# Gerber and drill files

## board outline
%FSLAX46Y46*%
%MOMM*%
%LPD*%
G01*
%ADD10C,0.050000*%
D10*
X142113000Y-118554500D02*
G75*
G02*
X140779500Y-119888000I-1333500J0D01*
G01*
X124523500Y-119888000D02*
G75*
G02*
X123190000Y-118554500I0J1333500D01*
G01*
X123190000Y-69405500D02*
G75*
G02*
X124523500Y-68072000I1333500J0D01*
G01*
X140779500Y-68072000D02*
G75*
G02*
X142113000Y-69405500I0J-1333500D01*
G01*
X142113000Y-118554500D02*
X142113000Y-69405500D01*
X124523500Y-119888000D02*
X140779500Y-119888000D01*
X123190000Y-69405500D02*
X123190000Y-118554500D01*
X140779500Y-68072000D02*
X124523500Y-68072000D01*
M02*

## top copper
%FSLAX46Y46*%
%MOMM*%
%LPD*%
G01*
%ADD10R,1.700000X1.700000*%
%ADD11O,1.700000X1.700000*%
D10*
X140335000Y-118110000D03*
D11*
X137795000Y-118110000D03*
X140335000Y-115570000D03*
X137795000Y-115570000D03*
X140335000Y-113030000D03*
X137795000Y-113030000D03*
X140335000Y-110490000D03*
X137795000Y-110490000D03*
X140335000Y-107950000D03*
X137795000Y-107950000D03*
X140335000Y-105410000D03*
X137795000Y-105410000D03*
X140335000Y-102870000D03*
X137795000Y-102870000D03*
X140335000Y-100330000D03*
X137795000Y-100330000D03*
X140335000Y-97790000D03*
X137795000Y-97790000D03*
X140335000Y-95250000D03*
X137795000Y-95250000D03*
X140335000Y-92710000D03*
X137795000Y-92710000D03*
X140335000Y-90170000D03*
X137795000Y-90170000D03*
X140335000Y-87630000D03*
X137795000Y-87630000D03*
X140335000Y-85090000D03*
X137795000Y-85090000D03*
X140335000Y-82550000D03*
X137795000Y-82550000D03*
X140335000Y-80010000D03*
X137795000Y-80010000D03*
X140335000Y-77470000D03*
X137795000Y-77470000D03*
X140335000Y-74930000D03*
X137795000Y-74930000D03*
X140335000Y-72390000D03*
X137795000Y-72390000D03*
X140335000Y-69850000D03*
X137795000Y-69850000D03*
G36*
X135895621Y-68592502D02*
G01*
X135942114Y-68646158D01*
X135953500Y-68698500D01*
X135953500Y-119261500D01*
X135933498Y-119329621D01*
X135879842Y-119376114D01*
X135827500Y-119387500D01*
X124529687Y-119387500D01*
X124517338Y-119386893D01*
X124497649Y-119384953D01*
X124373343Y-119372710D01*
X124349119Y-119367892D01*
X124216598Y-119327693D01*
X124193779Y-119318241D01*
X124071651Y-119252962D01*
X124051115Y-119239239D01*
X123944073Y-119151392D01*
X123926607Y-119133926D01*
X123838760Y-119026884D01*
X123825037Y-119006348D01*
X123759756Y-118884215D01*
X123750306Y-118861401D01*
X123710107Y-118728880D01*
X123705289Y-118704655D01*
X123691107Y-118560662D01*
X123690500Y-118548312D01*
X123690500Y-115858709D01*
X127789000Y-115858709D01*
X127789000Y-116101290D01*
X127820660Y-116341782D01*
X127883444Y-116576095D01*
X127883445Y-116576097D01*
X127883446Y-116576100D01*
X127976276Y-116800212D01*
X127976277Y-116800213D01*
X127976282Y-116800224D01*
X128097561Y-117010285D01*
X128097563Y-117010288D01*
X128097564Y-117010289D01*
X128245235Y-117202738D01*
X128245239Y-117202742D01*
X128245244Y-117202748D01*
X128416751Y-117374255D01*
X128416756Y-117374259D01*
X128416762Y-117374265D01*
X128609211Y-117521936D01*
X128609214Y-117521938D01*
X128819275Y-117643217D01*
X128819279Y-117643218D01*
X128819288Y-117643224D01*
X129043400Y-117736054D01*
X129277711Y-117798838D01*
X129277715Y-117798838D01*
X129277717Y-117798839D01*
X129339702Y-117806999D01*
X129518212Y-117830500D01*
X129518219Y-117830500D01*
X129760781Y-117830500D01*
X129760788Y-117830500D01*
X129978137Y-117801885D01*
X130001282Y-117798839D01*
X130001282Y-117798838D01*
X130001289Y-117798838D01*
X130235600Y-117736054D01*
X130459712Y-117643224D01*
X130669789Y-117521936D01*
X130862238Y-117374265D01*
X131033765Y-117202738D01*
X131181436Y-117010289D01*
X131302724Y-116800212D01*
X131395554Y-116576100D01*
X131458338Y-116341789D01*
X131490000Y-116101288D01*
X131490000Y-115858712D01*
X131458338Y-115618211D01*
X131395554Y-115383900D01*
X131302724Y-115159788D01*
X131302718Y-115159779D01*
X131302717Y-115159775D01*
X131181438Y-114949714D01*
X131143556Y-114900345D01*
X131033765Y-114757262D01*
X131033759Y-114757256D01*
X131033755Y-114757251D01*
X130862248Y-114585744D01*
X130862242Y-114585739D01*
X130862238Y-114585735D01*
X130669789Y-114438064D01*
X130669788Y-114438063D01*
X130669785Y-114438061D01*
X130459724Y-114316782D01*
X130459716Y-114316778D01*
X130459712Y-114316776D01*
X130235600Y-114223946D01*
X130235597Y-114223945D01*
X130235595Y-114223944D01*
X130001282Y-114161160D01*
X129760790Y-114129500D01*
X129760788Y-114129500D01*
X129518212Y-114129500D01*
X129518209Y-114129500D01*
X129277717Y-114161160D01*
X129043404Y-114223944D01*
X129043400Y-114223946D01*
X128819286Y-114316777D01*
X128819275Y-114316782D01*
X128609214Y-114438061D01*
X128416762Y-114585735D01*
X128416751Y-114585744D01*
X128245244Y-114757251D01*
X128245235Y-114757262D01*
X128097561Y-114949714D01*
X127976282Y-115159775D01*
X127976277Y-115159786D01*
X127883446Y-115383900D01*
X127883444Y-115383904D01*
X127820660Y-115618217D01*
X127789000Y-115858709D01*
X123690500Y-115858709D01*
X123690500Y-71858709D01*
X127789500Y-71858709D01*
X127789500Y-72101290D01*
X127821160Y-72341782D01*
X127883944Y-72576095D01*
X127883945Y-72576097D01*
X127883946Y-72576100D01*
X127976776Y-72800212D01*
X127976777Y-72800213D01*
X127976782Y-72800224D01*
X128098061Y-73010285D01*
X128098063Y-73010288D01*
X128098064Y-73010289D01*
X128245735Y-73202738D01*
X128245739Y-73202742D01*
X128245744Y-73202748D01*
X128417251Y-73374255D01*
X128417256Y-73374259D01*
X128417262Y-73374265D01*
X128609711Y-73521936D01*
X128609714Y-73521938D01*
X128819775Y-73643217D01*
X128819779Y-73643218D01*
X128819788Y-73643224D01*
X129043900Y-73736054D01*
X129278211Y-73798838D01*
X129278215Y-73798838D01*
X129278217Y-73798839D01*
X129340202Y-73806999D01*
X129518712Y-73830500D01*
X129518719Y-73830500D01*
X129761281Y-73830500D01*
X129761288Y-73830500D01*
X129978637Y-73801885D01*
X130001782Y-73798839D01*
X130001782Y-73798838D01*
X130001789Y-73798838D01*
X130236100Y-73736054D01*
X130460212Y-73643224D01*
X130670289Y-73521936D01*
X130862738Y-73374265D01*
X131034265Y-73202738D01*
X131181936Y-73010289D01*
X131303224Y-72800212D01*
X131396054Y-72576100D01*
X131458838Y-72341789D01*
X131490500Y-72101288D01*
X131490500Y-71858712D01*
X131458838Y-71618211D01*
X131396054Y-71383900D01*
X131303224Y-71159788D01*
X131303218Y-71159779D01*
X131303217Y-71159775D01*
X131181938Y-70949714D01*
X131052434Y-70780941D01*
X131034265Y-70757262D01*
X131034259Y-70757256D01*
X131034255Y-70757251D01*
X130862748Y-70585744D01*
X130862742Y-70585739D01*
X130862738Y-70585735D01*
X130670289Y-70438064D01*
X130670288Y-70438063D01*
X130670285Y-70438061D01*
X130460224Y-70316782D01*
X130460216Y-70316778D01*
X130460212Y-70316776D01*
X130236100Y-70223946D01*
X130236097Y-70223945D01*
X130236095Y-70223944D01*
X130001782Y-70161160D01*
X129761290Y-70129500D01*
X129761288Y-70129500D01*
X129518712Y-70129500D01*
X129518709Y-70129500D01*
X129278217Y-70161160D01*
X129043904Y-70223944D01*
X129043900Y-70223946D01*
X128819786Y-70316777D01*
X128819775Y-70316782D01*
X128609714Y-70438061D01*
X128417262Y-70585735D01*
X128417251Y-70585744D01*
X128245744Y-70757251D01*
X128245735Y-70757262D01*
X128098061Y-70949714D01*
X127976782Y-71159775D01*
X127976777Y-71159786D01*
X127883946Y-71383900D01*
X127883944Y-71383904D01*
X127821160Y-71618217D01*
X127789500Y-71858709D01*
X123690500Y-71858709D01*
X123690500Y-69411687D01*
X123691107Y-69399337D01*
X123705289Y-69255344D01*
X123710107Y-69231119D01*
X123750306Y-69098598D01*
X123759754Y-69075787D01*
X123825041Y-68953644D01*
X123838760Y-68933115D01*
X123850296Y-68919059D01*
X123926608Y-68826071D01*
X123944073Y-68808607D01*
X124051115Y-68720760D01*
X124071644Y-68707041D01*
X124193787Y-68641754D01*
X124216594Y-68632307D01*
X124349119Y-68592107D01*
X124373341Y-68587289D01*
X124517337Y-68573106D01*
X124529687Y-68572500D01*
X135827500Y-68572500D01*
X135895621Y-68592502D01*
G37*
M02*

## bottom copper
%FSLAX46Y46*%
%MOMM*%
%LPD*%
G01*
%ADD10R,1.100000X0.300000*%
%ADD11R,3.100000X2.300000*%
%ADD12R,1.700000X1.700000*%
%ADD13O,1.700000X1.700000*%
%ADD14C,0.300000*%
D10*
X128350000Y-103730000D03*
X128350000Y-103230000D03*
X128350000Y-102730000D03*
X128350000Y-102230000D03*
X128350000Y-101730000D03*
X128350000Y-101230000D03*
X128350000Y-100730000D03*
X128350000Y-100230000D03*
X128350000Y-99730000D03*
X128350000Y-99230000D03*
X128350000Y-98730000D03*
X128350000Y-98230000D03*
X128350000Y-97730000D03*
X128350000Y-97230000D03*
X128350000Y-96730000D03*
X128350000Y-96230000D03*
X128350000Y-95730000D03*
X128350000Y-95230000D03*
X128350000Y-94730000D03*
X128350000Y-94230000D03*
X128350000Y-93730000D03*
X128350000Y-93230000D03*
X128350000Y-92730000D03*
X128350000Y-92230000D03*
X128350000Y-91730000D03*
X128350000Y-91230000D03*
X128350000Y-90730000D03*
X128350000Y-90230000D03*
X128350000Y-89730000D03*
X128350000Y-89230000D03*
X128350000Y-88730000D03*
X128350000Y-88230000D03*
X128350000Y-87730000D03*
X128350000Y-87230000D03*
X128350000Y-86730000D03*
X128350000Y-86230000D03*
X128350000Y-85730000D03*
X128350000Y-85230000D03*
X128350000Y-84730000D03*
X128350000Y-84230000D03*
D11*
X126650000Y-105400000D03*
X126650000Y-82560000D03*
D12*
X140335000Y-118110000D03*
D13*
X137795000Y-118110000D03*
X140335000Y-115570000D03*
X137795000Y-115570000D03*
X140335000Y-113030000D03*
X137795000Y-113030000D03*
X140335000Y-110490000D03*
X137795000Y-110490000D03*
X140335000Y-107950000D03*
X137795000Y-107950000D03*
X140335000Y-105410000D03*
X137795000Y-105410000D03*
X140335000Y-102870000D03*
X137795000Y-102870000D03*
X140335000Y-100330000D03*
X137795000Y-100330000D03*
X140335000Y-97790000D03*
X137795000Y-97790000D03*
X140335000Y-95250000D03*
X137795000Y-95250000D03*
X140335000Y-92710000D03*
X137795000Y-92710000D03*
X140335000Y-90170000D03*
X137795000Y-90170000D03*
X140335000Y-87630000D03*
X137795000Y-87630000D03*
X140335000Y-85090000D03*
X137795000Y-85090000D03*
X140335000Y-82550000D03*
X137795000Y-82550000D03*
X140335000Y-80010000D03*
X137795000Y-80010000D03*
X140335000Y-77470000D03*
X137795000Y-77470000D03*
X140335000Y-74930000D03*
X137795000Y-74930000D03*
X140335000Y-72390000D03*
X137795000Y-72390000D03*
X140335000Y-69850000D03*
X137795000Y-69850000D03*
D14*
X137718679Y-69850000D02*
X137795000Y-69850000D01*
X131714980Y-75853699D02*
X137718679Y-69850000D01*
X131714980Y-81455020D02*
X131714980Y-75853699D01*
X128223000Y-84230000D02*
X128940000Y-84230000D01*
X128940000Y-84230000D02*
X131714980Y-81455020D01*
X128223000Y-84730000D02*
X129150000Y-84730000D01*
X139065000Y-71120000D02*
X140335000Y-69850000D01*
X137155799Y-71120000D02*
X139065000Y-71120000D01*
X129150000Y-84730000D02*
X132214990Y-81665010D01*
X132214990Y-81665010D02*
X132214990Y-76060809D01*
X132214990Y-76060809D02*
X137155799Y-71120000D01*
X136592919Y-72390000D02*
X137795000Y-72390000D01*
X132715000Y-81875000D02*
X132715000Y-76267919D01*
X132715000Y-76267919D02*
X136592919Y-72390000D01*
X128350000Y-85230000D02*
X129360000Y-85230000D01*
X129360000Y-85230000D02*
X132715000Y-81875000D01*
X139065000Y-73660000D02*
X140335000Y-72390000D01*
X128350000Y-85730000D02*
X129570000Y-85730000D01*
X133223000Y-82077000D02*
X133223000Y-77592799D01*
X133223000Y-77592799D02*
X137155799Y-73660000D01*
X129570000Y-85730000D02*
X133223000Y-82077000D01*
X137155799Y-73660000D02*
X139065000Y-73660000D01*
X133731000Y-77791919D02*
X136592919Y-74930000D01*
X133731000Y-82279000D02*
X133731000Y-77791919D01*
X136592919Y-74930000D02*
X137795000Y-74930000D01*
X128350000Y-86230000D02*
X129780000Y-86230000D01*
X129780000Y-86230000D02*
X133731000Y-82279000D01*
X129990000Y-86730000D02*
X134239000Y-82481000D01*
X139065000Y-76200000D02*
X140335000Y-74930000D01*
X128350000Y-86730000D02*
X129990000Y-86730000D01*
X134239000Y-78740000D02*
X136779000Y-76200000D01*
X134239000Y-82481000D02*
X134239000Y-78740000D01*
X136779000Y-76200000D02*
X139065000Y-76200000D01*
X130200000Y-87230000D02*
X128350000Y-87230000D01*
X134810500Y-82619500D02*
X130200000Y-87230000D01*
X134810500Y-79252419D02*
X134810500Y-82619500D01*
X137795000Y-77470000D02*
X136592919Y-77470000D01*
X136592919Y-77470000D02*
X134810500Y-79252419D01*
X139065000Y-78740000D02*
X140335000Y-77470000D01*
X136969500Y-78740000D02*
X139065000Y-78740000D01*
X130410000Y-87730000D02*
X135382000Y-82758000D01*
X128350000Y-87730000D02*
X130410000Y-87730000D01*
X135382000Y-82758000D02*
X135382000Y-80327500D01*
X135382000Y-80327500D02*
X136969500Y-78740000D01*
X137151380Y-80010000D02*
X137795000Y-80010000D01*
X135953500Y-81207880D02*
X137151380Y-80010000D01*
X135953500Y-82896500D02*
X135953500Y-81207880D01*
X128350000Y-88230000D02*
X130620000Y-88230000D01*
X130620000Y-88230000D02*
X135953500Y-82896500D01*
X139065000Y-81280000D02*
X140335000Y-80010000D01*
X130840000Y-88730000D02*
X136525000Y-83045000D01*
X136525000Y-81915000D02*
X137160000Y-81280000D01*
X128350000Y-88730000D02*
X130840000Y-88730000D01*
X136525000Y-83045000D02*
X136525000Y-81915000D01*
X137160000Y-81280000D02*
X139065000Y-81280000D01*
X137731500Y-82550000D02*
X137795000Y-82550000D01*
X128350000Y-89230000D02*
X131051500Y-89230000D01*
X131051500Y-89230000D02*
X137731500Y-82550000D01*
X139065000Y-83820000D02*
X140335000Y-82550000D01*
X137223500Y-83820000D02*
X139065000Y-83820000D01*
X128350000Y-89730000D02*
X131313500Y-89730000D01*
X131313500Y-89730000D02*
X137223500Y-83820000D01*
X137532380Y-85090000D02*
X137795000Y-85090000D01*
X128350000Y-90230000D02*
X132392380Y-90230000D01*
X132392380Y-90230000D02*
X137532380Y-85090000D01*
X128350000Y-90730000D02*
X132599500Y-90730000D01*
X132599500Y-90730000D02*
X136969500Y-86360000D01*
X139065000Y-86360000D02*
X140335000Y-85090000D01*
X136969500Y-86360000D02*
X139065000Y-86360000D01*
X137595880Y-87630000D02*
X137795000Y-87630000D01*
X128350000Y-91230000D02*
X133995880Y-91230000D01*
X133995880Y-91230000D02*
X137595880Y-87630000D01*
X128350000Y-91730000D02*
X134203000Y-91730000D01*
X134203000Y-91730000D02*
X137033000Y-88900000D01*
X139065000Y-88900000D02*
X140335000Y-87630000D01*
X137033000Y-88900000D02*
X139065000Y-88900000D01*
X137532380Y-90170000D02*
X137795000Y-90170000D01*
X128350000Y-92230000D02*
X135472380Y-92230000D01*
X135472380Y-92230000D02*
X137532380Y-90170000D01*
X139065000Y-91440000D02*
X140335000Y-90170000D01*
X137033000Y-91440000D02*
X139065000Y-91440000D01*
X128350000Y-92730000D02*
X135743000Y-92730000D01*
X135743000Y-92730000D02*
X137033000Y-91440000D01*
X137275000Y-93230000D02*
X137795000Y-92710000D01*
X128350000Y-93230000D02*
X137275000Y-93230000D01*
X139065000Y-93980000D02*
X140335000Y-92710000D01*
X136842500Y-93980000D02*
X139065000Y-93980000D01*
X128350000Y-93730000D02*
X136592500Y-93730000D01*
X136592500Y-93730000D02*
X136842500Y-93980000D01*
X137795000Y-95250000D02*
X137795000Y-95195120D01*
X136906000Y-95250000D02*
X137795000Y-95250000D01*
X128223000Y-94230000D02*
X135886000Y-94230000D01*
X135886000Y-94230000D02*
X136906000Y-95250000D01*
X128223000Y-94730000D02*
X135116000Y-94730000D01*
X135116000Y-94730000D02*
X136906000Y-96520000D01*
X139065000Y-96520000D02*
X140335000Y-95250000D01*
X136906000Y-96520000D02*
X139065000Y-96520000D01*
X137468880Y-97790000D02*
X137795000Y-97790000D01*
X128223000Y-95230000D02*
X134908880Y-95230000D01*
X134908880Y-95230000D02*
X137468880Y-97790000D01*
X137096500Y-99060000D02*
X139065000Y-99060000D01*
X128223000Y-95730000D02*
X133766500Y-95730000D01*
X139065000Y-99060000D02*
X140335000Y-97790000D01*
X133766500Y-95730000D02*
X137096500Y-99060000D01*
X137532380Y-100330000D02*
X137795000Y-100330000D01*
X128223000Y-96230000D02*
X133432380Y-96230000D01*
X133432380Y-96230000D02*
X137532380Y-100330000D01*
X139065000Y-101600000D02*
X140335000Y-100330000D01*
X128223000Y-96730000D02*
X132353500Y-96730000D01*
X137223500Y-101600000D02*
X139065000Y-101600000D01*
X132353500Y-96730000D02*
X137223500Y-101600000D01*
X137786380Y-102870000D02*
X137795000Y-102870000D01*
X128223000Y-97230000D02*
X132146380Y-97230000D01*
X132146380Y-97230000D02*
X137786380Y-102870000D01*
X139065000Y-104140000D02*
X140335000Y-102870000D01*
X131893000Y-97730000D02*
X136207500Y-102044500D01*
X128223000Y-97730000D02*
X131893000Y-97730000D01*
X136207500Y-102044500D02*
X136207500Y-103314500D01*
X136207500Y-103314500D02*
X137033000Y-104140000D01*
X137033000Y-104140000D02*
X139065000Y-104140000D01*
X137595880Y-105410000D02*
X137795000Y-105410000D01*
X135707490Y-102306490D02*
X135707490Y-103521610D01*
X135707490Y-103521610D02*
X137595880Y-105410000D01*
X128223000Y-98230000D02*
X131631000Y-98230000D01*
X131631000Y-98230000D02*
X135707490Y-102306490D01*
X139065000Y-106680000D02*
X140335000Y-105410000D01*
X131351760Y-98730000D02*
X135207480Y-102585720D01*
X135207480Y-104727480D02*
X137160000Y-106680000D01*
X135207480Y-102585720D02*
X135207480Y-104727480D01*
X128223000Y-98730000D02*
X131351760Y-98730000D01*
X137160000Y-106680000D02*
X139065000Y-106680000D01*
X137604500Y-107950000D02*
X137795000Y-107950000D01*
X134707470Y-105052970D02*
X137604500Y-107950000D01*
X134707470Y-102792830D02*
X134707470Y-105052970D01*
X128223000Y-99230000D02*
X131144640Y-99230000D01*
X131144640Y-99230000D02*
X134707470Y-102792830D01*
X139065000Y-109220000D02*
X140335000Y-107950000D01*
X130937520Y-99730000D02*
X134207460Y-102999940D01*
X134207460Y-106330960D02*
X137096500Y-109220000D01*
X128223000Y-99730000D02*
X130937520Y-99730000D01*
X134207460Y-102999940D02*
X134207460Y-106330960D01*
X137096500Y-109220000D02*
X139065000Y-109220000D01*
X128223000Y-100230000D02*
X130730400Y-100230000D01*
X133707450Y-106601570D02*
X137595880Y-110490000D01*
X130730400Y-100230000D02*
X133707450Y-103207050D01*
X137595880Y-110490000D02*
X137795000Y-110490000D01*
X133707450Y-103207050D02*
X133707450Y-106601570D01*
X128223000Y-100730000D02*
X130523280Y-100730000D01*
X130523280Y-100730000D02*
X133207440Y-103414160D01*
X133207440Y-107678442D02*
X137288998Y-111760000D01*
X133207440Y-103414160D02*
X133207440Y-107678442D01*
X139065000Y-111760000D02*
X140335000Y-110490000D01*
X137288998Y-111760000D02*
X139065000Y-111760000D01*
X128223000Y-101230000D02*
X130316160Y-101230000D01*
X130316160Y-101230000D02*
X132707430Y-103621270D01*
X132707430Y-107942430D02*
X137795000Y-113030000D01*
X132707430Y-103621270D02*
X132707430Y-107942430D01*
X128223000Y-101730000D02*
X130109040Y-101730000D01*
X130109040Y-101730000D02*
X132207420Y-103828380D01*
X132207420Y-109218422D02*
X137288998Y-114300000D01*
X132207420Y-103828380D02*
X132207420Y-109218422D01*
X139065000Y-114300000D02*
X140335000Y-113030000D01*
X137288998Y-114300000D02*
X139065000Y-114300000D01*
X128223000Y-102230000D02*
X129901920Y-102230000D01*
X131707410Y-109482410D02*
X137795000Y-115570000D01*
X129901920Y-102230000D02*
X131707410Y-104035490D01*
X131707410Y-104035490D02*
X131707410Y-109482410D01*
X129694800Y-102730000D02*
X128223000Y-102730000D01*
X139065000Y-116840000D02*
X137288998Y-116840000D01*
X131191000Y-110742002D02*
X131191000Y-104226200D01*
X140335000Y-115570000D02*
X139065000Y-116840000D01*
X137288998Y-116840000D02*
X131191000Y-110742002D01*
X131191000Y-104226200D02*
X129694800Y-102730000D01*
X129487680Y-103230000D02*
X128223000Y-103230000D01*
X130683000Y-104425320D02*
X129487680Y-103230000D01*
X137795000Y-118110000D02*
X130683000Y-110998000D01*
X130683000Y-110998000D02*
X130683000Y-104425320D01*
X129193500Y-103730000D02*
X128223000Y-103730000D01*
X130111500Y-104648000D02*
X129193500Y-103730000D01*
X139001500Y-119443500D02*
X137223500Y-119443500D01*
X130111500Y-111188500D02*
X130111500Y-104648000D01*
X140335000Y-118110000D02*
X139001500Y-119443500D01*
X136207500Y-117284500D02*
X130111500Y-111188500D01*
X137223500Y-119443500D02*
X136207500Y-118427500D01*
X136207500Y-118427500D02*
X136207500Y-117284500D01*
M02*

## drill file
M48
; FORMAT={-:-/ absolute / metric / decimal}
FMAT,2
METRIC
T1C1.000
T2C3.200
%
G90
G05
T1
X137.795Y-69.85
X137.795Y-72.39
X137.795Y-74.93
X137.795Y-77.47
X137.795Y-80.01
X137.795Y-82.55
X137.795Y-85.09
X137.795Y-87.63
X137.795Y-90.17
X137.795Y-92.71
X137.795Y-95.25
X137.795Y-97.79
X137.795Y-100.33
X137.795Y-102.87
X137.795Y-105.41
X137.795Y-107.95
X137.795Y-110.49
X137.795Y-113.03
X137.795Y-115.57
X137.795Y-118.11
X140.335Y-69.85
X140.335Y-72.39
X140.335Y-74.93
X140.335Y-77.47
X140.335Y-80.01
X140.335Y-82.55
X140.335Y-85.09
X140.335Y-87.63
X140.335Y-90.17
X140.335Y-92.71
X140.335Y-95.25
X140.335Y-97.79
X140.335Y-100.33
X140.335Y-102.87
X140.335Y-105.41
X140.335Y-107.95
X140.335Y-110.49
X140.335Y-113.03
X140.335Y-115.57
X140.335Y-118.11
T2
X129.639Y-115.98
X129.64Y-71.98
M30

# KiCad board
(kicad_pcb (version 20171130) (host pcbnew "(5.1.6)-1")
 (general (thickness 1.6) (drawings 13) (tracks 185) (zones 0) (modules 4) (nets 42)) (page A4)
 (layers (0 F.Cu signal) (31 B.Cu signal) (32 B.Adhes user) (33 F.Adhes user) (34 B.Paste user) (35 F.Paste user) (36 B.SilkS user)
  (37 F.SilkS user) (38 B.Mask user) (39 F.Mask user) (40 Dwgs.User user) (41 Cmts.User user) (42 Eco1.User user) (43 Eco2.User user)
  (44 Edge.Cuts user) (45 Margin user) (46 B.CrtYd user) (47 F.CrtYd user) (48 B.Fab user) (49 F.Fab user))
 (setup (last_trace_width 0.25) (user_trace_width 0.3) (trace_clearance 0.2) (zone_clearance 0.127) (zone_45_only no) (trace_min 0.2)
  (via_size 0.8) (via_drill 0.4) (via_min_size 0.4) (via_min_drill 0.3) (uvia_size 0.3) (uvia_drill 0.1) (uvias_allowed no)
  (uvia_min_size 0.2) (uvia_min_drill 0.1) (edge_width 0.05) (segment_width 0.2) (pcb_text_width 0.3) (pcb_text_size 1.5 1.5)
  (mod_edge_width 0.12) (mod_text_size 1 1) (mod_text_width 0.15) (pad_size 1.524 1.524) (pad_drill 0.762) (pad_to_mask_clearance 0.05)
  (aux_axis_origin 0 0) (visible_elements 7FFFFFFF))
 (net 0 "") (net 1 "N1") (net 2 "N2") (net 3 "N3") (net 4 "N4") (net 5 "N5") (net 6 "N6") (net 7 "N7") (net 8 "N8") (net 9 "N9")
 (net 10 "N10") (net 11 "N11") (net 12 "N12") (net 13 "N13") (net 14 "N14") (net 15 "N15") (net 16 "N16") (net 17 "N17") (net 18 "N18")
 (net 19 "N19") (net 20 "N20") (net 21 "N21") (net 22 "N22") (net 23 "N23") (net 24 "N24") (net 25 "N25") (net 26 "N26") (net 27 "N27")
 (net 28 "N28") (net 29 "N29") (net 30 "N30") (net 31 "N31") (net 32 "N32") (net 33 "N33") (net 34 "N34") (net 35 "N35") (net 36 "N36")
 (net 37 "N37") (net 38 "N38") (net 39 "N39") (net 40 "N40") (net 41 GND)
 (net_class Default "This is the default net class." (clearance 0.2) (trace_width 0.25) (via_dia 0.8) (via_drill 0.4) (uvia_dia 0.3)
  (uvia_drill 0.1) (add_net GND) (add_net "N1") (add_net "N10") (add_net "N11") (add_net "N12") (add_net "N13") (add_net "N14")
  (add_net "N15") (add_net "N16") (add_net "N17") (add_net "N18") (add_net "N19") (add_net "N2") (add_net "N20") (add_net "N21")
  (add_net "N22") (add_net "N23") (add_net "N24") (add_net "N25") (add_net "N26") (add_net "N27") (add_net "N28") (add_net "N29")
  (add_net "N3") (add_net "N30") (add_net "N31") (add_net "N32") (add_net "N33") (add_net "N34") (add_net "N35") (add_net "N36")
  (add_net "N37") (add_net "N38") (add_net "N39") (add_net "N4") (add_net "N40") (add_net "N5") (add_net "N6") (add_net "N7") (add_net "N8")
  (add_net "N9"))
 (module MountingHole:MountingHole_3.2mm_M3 (layer F.Cu) (at 129.64 71.98)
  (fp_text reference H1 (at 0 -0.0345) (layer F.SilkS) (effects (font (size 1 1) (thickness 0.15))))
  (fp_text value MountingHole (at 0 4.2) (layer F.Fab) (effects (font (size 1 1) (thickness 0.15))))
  (pad 1 np_thru_hole circle (at 0 0) (size 3.2 3.2) (drill 3.2) (layers *.Cu *.Mask)))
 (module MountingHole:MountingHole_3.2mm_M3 (layer F.Cu) (at 129.6395 115.98)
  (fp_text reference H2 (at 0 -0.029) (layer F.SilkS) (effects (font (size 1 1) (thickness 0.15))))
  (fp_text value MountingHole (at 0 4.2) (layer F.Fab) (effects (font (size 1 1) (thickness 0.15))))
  (pad 1 np_thru_hole circle (at 0 0) (size 3.2 3.2) (drill 3.2) (layers *.Cu *.Mask)))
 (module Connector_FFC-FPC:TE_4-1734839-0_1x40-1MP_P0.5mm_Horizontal (layer B.Cu) (at 127 93.98 90)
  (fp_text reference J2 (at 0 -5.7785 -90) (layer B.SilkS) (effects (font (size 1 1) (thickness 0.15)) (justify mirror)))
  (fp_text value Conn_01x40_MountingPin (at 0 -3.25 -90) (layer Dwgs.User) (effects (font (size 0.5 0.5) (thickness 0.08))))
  (pad 1 smd rect (at -9.75 1.35 90) (size 0.3 1.1) (layers B.Cu B.Paste B.Mask) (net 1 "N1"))
  (pad 2 smd rect (at -9.25 1.35 90) (size 0.3 1.1) (layers B.Cu B.Paste B.Mask) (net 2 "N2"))
  (pad 3 smd rect (at -8.75 1.35 90) (size 0.3 1.1) (layers B.Cu B.Paste B.Mask) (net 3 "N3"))
  (pad 4 smd rect (at -8.25 1.35 90) (size 0.3 1.1) (layers B.Cu B.Paste B.Mask) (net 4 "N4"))
  (pad 5 smd rect (at -7.75 1.35 90) (size 0.3 1.1) (layers B.Cu B.Paste B.Mask) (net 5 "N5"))
  (pad 6 smd rect (at -7.25 1.35 90) (size 0.3 1.1) (layers B.Cu B.Paste B.Mask) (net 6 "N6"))
  (pad 7 smd rect (at -6.75 1.35 90) (size 0.3 1.1) (layers B.Cu B.Paste B.Mask) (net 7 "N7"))
  (pad 8 smd rect (at -6.25 1.35 90) (size 0.3 1.1) (layers B.Cu B.Paste B.Mask) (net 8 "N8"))
  (pad 9 smd rect (at -5.75 1.35 90) (size 0.3 1.1) (layers B.Cu B.Paste B.Mask) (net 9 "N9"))
  (pad 10 smd rect (at -5.25 1.35 90) (size 0.3 1.1) (layers B.Cu B.Paste B.Mask) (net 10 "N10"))
  (pad 11 smd rect (at -4.75 1.35 90) (size 0.3 1.1) (layers B.Cu B.Paste B.Mask) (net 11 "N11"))
  (pad 12 smd rect (at -4.25 1.35 90) (size 0.3 1.1) (layers B.Cu B.Paste B.Mask) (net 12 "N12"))
  (pad 13 smd rect (at -3.75 1.35 90) (size 0.3 1.1) (layers B.Cu B.Paste B.Mask) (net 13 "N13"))
  (pad 14 smd rect (at -3.25 1.35 90) (size 0.3 1.1) (layers B.Cu B.Paste B.Mask) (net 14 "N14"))
  (pad 15 smd rect (at -2.75 1.35 90) (size 0.3 1.1) (layers B.Cu B.Paste B.Mask) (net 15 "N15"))
  (pad 16 smd rect (at -2.25 1.35 90) (size 0.3 1.1) (layers B.Cu B.Paste B.Mask) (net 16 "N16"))
  (pad 17 smd rect (at -1.75 1.35 90) (size 0.3 1.1) (layers B.Cu B.Paste B.Mask) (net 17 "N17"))
  (pad 18 smd rect (at -1.25 1.35 90) (size 0.3 1.1) (layers B.Cu B.Paste B.Mask) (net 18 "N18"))
  (pad 19 smd rect (at -0.75 1.35 90) (size 0.3 1.1) (layers B.Cu B.Paste B.Mask) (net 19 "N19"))
  (pad 20 smd rect (at -0.25 1.35 90) (size 0.3 1.1) (layers B.Cu B.Paste B.Mask) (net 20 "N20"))
  (pad 21 smd rect (at 0.25 1.35 90) (size 0.3 1.1) (layers B.Cu B.Paste B.Mask) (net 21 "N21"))
  (pad 22 smd rect (at 0.75 1.35 90) (size 0.3 1.1) (layers B.Cu B.Paste B.Mask) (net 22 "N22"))
  (pad 23 smd rect (at 1.25 1.35 90) (size 0.3 1.1) (layers B.Cu B.Paste B.Mask) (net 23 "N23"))
  (pad 24 smd rect (at 1.75 1.35 90) (size 0.3 1.1) (layers B.Cu B.Paste B.Mask) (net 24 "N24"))
  (pad 25 smd rect (at 2.25 1.35 90) (size 0.3 1.1) (layers B.Cu B.Paste B.Mask) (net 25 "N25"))
  (pad 26 smd rect (at 2.75 1.35 90) (size 0.3 1.1) (layers B.Cu B.Paste B.Mask) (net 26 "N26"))
  (pad 27 smd rect (at 3.25 1.35 90) (size 0.3 1.1) (layers B.Cu B.Paste B.Mask) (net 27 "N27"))
  (pad 28 smd rect (at 3.75 1.35 90) (size 0.3 1.1) (layers B.Cu B.Paste B.Mask) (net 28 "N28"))
  (pad 29 smd rect (at 4.25 1.35 90) (size 0.3 1.1) (layers B.Cu B.Paste B.Mask) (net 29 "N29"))
  (pad 30 smd rect (at 4.75 1.35 90) (size 0.3 1.1) (layers B.Cu B.Paste B.Mask) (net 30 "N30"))
  (pad 31 smd rect (at 5.25 1.35 90) (size 0.3 1.1) (layers B.Cu B.Paste B.Mask) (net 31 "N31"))
  (pad 32 smd rect (at 5.75 1.35 90) (size 0.3 1.1) (layers B.Cu B.Paste B.Mask) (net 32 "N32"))
  (pad 33 smd rect (at 6.25 1.35 90) (size 0.3 1.1) (layers B.Cu B.Paste B.Mask) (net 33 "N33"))
  (pad 34 smd rect (at 6.75 1.35 90) (size 0.3 1.1) (layers B.Cu B.Paste B.Mask) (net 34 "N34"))
  (pad 35 smd rect (at 7.25 1.35 90) (size 0.3 1.1) (layers B.Cu B.Paste B.Mask) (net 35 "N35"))
  (pad 36 smd rect (at 7.75 1.35 90) (size 0.3 1.1) (layers B.Cu B.Paste B.Mask) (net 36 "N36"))
  (pad 37 smd rect (at 8.25 1.35 90) (size 0.3 1.1) (layers B.Cu B.Paste B.Mask) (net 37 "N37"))
  (pad 38 smd rect (at 8.75 1.35 90) (size 0.3 1.1) (layers B.Cu B.Paste B.Mask) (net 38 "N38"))
  (pad 39 smd rect (at 9.25 1.35 90) (size 0.3 1.1) (layers B.Cu B.Paste B.Mask) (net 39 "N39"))
  (pad 40 smd rect (at 9.75 1.35 90) (size 0.3 1.1) (layers B.Cu B.Paste B.Mask) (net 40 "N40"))
  (pad MP smd rect (at -11.42 -0.35 90) (size 2.3 3.1) (layers B.Cu B.Paste B.Mask) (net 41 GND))
  (pad MP smd rect (at 11.42 -0.35 90) (size 2.3 3.1) (layers B.Cu B.Paste B.Mask) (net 41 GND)))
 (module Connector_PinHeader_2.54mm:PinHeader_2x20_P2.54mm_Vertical (layer F.Cu) (at 140.335 118.11 180)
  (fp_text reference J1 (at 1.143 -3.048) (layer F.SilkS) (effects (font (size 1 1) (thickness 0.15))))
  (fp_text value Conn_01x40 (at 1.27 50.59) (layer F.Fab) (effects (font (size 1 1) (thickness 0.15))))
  (pad 1 thru_hole rect (at 0 0 180) (size 1.7 1.7) (drill 1) (layers *.Cu *.Mask) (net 1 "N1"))
  (pad 2 thru_hole oval (at 2.54 0 180) (size 1.7 1.7) (drill 1) (layers *.Cu *.Mask) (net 2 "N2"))
  (pad 3 thru_hole oval (at 0 2.54 180) (size 1.7 1.7) (drill 1) (layers *.Cu *.Mask) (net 3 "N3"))
  (pad 4 thru_hole oval (at 2.54 2.54 180) (size 1.7 1.7) (drill 1) (layers *.Cu *.Mask) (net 4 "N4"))
  (pad 5 thru_hole oval (at 0 5.08 180) (size 1.7 1.7) (drill 1) (layers *.Cu *.Mask) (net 5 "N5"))
  (pad 6 thru_hole oval (at 2.54 5.08 180) (size 1.7 1.7) (drill 1) (layers *.Cu *.Mask) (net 6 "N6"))
  (pad 7 thru_hole oval (at 0 7.62 180) (size 1.7 1.7) (drill 1) (layers *.Cu *.Mask) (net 7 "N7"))
  (pad 8 thru_hole oval (at 2.54 7.62 180) (size 1.7 1.7) (drill 1) (layers *.Cu *.Mask) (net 8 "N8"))
  (pad 9 thru_hole oval (at 0 10.16 180) (size 1.7 1.7) (drill 1) (layers *.Cu *.Mask) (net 9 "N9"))
  (pad 10 thru_hole oval (at 2.54 10.16 180) (size 1.7 1.7) (drill 1) (layers *.Cu *.Mask) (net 10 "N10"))
  (pad 11 thru_hole oval (at 0 12.7 180) (size 1.7 1.7) (drill 1) (layers *.Cu *.Mask) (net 11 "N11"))
  (pad 12 thru_hole oval (at 2.54 12.7 180) (size 1.7 1.7) (drill 1) (layers *.Cu *.Mask) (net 12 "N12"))
  (pad 13 thru_hole oval (at 0 15.24 180) (size 1.7 1.7) (drill 1) (layers *.Cu *.Mask) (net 13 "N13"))
  (pad 14 thru_hole oval (at 2.54 15.24 180) (size 1.7 1.7) (drill 1) (layers *.Cu *.Mask) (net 14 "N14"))
  (pad 15 thru_hole oval (at 0 17.78 180) (size 1.7 1.7) (drill 1) (layers *.Cu *.Mask) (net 15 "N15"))
  (pad 16 thru_hole oval (at 2.54 17.78 180) (size 1.7 1.7) (drill 1) (layers *.Cu *.Mask) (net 16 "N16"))
  (pad 17 thru_hole oval (at 0 20.32 180) (size 1.7 1.7) (drill 1) (layers *.Cu *.Mask) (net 17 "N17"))
  (pad 18 thru_hole oval (at 2.54 20.32 180) (size 1.7 1.7) (drill 1) (layers *.Cu *.Mask) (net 18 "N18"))
  (pad 19 thru_hole oval (at 0 22.86 180) (size 1.7 1.7) (drill 1) (layers *.Cu *.Mask) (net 19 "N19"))
  (pad 20 thru_hole oval (at 2.54 22.86 180) (size 1.7 1.7) (drill 1) (layers *.Cu *.Mask) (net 20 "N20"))
  (pad 21 thru_hole oval (at 0 25.4 180) (size 1.7 1.7) (drill 1) (layers *.Cu *.Mask) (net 21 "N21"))
  (pad 22 thru_hole oval (at 2.54 25.4 180) (size 1.7 1.7) (drill 1) (layers *.Cu *.Mask) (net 22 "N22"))
  (pad 23 thru_hole oval (at 0 27.94 180) (size 1.7 1.7) (drill 1) (layers *.Cu *.Mask) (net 23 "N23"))
  (pad 24 thru_hole oval (at 2.54 27.94 180) (size 1.7 1.7) (drill 1) (layers *.Cu *.Mask) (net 24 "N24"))
  (pad 25 thru_hole oval (at 0 30.48 180) (size 1.7 1.7) (drill 1) (layers *.Cu *.Mask) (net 25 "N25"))
  (pad 26 thru_hole oval (at 2.54 30.48 180) (size 1.7 1.7) (drill 1) (layers *.Cu *.Mask) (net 26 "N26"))
  (pad 27 thru_hole oval (at 0 33.02 180) (size 1.7 1.7) (drill 1) (layers *.Cu *.Mask) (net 27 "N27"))
  (pad 28 thru_hole oval (at 2.54 33.02 180) (size 1.7 1.7) (drill 1) (layers *.Cu *.Mask) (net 28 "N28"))
  (pad 29 thru_hole oval (at 0 35.56 180) (size 1.7 1.7) (drill 1) (layers *.Cu *.Mask) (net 29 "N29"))
  (pad 30 thru_hole oval (at 2.54 35.56 180) (size 1.7 1.7) (drill 1) (layers *.Cu *.Mask) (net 30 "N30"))
  (pad 31 thru_hole oval (at 0 38.1 180) (size 1.7 1.7) (drill 1) (layers *.Cu *.Mask) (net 31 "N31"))
  (pad 32 thru_hole oval (at 2.54 38.1 180) (size 1.7 1.7) (drill 1) (layers *.Cu *.Mask) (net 32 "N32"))
  (pad 33 thru_hole oval (at 0 40.64 180) (size 1.7 1.7) (drill 1) (layers *.Cu *.Mask) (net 33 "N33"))
  (pad 34 thru_hole oval (at 2.54 40.64 180) (size 1.7 1.7) (drill 1) (layers *.Cu *.Mask) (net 34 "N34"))
  (pad 35 thru_hole oval (at 0 43.18 180) (size 1.7 1.7) (drill 1) (layers *.Cu *.Mask) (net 35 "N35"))
  (pad 36 thru_hole oval (at 2.54 43.18 180) (size 1.7 1.7) (drill 1) (layers *.Cu *.Mask) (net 36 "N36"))
  (pad 37 thru_hole oval (at 0 45.72 180) (size 1.7 1.7) (drill 1) (layers *.Cu *.Mask) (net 37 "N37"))
  (pad 38 thru_hole oval (at 2.54 45.72 180) (size 1.7 1.7) (drill 1) (layers *.Cu *.Mask) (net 38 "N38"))
  (pad 39 thru_hole oval (at 0 48.26 180) (size 1.7 1.7) (drill 1) (layers *.Cu *.Mask) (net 39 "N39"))
  (pad 40 thru_hole oval (at 2.54 48.26 180) (size 1.7 1.7) (drill 1) (layers *.Cu *.Mask) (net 40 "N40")))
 (gr_arc (start 140.7795 118.5545) (end 140.7795 119.888) (angle -90) (layer Edge.Cuts) (width 0.05))
 (gr_arc (start 124.5235 118.5545) (end 123.19 118.5545) (angle -90) (layer Edge.Cuts) (width 0.05))
 (gr_arc (start 124.5235 69.4055) (end 124.5235 68.072) (angle -90) (layer Edge.Cuts) (width 0.05))
 (gr_arc (start 140.7795 69.4055) (end 142.113 69.4055) (angle -90) (layer Edge.Cuts) (width 0.05))
 (gr_line (start 142.113 118.5545) (end 142.113 69.4055) (layer Edge.Cuts) (width 0.05))
 (gr_line (start 124.5235 119.888) (end 140.7795 119.888) (layer Edge.Cuts) (width 0.05))
 (gr_line (start 123.19 69.4055) (end 123.19 118.5545) (layer Edge.Cuts) (width 0.05))
 (gr_line (start 140.7795 68.072) (end 124.5235 68.072) (layer Edge.Cuts) (width 0.05))
 (segment (start 137.718679 69.85) (end 137.795 69.85) (width 0.3) (layer B.Cu) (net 40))
 (segment (start 131.71498 75.853699) (end 137.718679 69.85) (width 0.3) (layer B.Cu) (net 40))
 (segment (start 131.71498 81.45502) (end 131.71498 75.853699) (width 0.3) (layer B.Cu) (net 40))
 (segment (start 128.223 84.23) (end 128.94 84.23) (width 0.3) (layer B.Cu) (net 40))
 (segment (start 128.94 84.23) (end 131.71498 81.45502) (width 0.3) (layer B.Cu) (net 40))
 (segment (start 128.223 84.73) (end 129.15 84.73) (width 0.3) (layer B.Cu) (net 39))
 (segment (start 139.065 71.12) (end 140.335 69.85) (width 0.3) (layer B.Cu) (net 39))
 (segment (start 137.155799 71.12) (end 139.065 71.12) (width 0.3) (layer B.Cu) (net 39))
 (segment (start 129.15 84.73) (end 132.21499 81.66501) (width 0.3) (layer B.Cu) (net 39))
 (segment (start 132.21499 81.66501) (end 132.21499 76.060809) (width 0.3) (layer B.Cu) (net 39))
 (segment (start 132.21499 76.060809) (end 137.155799 71.12) (width 0.3) (layer B.Cu) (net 39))
 (segment (start 136.592919 72.39) (end 137.795 72.39) (width 0.3) (layer B.Cu) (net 38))
 (segment (start 132.715 81.875) (end 132.715 76.267919) (width 0.3) (layer B.Cu) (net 38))
 (segment (start 132.715 76.267919) (end 136.592919 72.39) (width 0.3) (layer B.Cu) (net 38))
 (segment (start 128.35 85.23) (end 129.36 85.23) (width 0.3) (layer B.Cu) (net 38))
 (segment (start 129.36 85.23) (end 132.715 81.875) (width 0.3) (layer B.Cu) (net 38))
 (segment (start 139.065 73.66) (end 140.335 72.39) (width 0.3) (layer B.Cu) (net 37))
 (segment (start 128.35 85.73) (end 129.57 85.73) (width 0.3) (layer B.Cu) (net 37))
 (segment (start 133.223 82.077) (end 133.223 77.592799) (width 0.3) (layer B.Cu) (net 37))
 (segment (start 133.223 77.592799) (end 137.155799 73.66) (width 0.3) (layer B.Cu) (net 37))
 (segment (start 129.57 85.73) (end 133.223 82.077) (width 0.3) (layer B.Cu) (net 37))
 (segment (start 137.155799 73.66) (end 139.065 73.66) (width 0.3) (layer B.Cu) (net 37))
 (segment (start 133.731 77.791919) (end 136.592919 74.93) (width 0.3) (layer B.Cu) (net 36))
 (segment (start 133.731 82.279) (end 133.731 77.791919) (width 0.3) (layer B.Cu) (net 36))
 (segment (start 136.592919 74.93) (end 137.795 74.93) (width 0.3) (layer B.Cu) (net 36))
 (segment (start 128.35 86.23) (end 129.78 86.23) (width 0.3) (layer B.Cu) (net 36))
 (segment (start 129.78 86.23) (end 133.731 82.279) (width 0.3) (layer B.Cu) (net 36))
 (segment (start 129.99 86.73) (end 134.239 82.481) (width 0.3) (layer B.Cu) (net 35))
 (segment (start 139.065 76.2) (end 140.335 74.93) (width 0.3) (layer B.Cu) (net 35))
 (segment (start 128.35 86.73) (end 129.99 86.73) (width 0.3) (layer B.Cu) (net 35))
 (segment (start 134.239 78.74) (end 136.779 76.2) (width 0.3) (layer B.Cu) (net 35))
 (segment (start 134.239 82.481) (end 134.239 78.74) (width 0.3) (layer B.Cu) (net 35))
 (segment (start 136.779 76.2) (end 139.065 76.2) (width 0.3) (layer B.Cu) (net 35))
 (segment (start 130.2 87.23) (end 128.35 87.23) (width 0.3) (layer B.Cu) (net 34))
 (segment (start 134.8105 82.6195) (end 130.2 87.23) (width 0.3) (layer B.Cu) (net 34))
 (segment (start 134.8105 79.252419) (end 134.8105 82.6195) (width 0.3) (layer B.Cu) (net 34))
 (segment (start 137.795 77.47) (end 136.592919 77.47) (width 0.3) (layer B.Cu) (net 34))
 (segment (start 136.592919 77.47) (end 134.8105 79.252419) (width 0.3) (layer B.Cu) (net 34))
 (segment (start 139.065 78.74) (end 140.335 77.47) (width 0.3) (layer B.Cu) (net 33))
 (segment (start 136.9695 78.74) (end 139.065 78.74) (width 0.3) (layer B.Cu) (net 33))
 (segment (start 130.41 87.73) (end 135.382 82.758) (width 0.3) (layer B.Cu) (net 33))
 (segment (start 128.35 87.73) (end 130.41 87.73) (width 0.3) (layer B.Cu) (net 33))
 (segment (start 135.382 82.758) (end 135.382 80.3275) (width 0.3) (layer B.Cu) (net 33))
 (segment (start 135.382 80.3275) (end 136.9695 78.74) (width 0.3) (layer B.Cu) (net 33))
 (segment (start 137.15138 80.01) (end 137.795 80.01) (width 0.3) (layer B.Cu) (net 32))
 (segment (start 135.9535 81.20788) (end 137.15138 80.01) (width 0.3) (layer B.Cu) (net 32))
 (segment (start 135.9535 82.8965) (end 135.9535 81.20788) (width 0.3) (layer B.Cu) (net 32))
 (segment (start 128.35 88.23) (end 130.62 88.23) (width 0.3) (layer B.Cu) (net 32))
 (segment (start 130.62 88.23) (end 135.9535 82.8965) (width 0.3) (layer B.Cu) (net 32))
 (segment (start 139.065 81.28) (end 140.335 80.01) (width 0.3) (layer B.Cu) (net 31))
 (segment (start 130.84 88.73) (end 136.525 83.045) (width 0.3) (layer B.Cu) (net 31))
 (segment (start 136.525 81.915) (end 137.16 81.28) (width 0.3) (layer B.Cu) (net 31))
 (segment (start 128.35 88.73) (end 130.84 88.73) (width 0.3) (layer B.Cu) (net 31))
 (segment (start 136.525 83.045) (end 136.525 81.915) (width 0.3) (layer B.Cu) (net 31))
 (segment (start 137.16 81.28) (end 139.065 81.28) (width 0.3) (layer B.Cu) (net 31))
 (segment (start 137.7315 82.55) (end 137.795 82.55) (width 0.3) (layer B.Cu) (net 30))
 (segment (start 128.35 89.23) (end 131.0515 89.23) (width 0.3) (layer B.Cu) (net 30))
 (segment (start 131.0515 89.23) (end 137.7315 82.55) (width 0.3) (layer B.Cu) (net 30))
 (segment (start 139.065 83.82) (end 140.335 82.55) (width 0.3) (layer B.Cu) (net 29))
 (segment (start 137.2235 83.82) (end 139.065 83.82) (width 0.3) (layer B.Cu) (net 29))
 (segment (start 128.35 89.73) (end 131.3135 89.73) (width 0.3) (layer B.Cu) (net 29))
 (segment (start 131.3135 89.73) (end 137.2235 83.82) (width 0.3) (layer B.Cu) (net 29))
 (segment (start 137.53238 85.09) (end 137.795 85.09) (width 0.3) (layer B.Cu) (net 28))
 (segment (start 128.35 90.23) (end 132.39238 90.23) (width 0.3) (layer B.Cu) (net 28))
 (segment (start 132.39238 90.23) (end 137.53238 85.09) (width 0.3) (layer B.Cu) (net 28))
 (segment (start 128.35 90.73) (end 132.5995 90.73) (width 0.3) (layer B.Cu) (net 27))
 (segment (start 132.5995 90.73) (end 136.9695 86.36) (width 0.3) (layer B.Cu) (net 27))
 (segment (start 139.065 86.36) (end 140.335 85.09) (width 0.3) (layer B.Cu) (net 27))
 (segment (start 136.9695 86.36) (end 139.065 86.36) (width 0.3) (layer B.Cu) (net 27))
 (segment (start 137.59588 87.63) (end 137.795 87.63) (width 0.3) (layer B.Cu) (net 26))
 (segment (start 128.35 91.23) (end 133.99588 91.23) (width 0.3) (layer B.Cu) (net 26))
 (segment (start 133.99588 91.23) (end 137.59588 87.63) (width 0.3) (layer B.Cu) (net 26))
 (segment (start 128.35 91.73) (end 134.203 91.73) (width 0.3) (layer B.Cu) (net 25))
 (segment (start 134.203 91.73) (end 137.033 88.9) (width 0.3) (layer B.Cu) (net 25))
 (segment (start 139.065 88.9) (end 140.335 87.63) (width 0.3) (layer B.Cu) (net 25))
 (segment (start 137.033 88.9) (end 139.065 88.9) (width 0.3) (layer B.Cu) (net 25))
 (segment (start 137.53238 90.17) (end 137.795 90.17) (width 0.3) (layer B.Cu) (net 24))
 (segment (start 128.35 92.23) (end 135.47238 92.23) (width 0.3) (layer B.Cu) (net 24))
 (segment (start 135.47238 92.23) (end 137.53238 90.17) (width 0.3) (layer B.Cu) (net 24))
 (segment (start 139.065 91.44) (end 140.335 90.17) (width 0.3) (layer B.Cu) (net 23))
 (segment (start 137.033 91.44) (end 139.065 91.44) (width 0.3) (layer B.Cu) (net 23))
 (segment (start 128.35 92.73) (end 135.743 92.73) (width 0.3) (layer B.Cu) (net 23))
 (segment (start 135.743 92.73) (end 137.033 91.44) (width 0.3) (layer B.Cu) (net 23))
 (segment (start 137.275 93.23) (end 137.795 92.71) (width 0.3) (layer B.Cu) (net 22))
 (segment (start 128.35 93.23) (end 137.275 93.23) (width 0.3) (layer B.Cu) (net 22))
 (segment (start 139.065 93.98) (end 140.335 92.71) (width 0.3) (layer B.Cu) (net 21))
 (segment (start 136.8425 93.98) (end 139.065 93.98) (width 0.3) (layer B.Cu) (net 21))
 (segment (start 128.35 93.73) (end 136.5925 93.73) (width 0.3) (layer B.Cu) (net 21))
 (segment (start 136.5925 93.73) (end 136.8425 93.98) (width 0.3) (layer B.Cu) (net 21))
 (segment (start 137.795 95.25) (end 137.795 95.19512) (width 0.3) (layer B.Cu) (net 20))
 (segment (start 136.906 95.25) (end 137.795 95.25) (width 0.3) (layer B.Cu) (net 20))
 (segment (start 128.223 94.23) (end 135.886 94.23) (width 0.3) (layer B.Cu) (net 20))
 (segment (start 135.886 94.23) (end 136.906 95.25) (width 0.3) (layer B.Cu) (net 20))
 (segment (start 128.223 94.73) (end 135.116 94.73) (width 0.3) (layer B.Cu) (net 19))
 (segment (start 135.116 94.73) (end 136.906 96.52) (width 0.3) (layer B.Cu) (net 19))
 (segment (start 139.065 96.52) (end 140.335 95.25) (width 0.3) (layer B.Cu) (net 19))
 (segment (start 136.906 96.52) (end 139.065 96.52) (width 0.3) (layer B.Cu) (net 19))
 (segment (start 137.46888 97.79) (end 137.795 97.79) (width 0.3) (layer B.Cu) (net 18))
 (segment (start 128.223 95.23) (end 134.90888 95.23) (width 0.3) (layer B.Cu) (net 18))
 (segment (start 134.90888 95.23) (end 137.46888 97.79) (width 0.3) (layer B.Cu) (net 18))
 (segment (start 137.0965 99.06) (end 139.065 99.06) (width 0.3) (layer B.Cu) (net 17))
 (segment (start 128.223 95.73) (end 133.7665 95.73) (width 0.3) (layer B.Cu) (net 17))
 (segment (start 139.065 99.06) (end 140.335 97.79) (width 0.3) (layer B.Cu) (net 17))
 (segment (start 133.7665 95.73) (end 137.0965 99.06) (width 0.3) (layer B.Cu) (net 17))
 (segment (start 137.53238 100.33) (end 137.795 100.33) (width 0.3) (layer B.Cu) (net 16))
 (segment (start 128.223 96.23) (end 133.43238 96.23) (width 0.3) (layer B.Cu) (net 16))
 (segment (start 133.43238 96.23) (end 137.53238 100.33) (width 0.3) (layer B.Cu) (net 16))
 (segment (start 139.065 101.6) (end 140.335 100.33) (width 0.3) (layer B.Cu) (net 15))
 (segment (start 128.223 96.73) (end 132.3535 96.73) (width 0.3) (layer B.Cu) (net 15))
 (segment (start 137.2235 101.6) (end 139.065 101.6) (width 0.3) (layer B.Cu) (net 15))
 (segment (start 132.3535 96.73) (end 137.2235 101.6) (width 0.3) (layer B.Cu) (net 15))
 (segment (start 137.78638 102.87) (end 137.795 102.87) (width 0.3) (layer B.Cu) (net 14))
 (segment (start 128.223 97.23) (end 132.14638 97.23) (width 0.3) (layer B.Cu) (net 14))
 (segment (start 132.14638 97.23) (end 137.78638 102.87) (width 0.3) (layer B.Cu) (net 14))
 (segment (start 139.065 104.14) (end 140.335 102.87) (width 0.3) (layer B.Cu) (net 13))
 (segment (start 131.893 97.73) (end 136.2075 102.0445) (width 0.3) (layer B.Cu) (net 13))
 (segment (start 128.223 97.73) (end 131.893 97.73) (width 0.3) (layer B.Cu) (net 13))
 (segment (start 136.2075 102.0445) (end 136.2075 103.3145) (width 0.3) (layer B.Cu) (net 13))
 (segment (start 136.2075 103.3145) (end 137.033 104.14) (width 0.3) (layer B.Cu) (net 13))
 (segment (start 137.033 104.14) (end 139.065 104.14) (width 0.3) (layer B.Cu) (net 13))
 (segment (start 137.59588 105.41) (end 137.795 105.41) (width 0.3) (layer B.Cu) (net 12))
 (segment (start 135.70749 102.30649) (end 135.70749 103.52161) (width 0.3) (layer B.Cu) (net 12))
 (segment (start 135.70749 103.52161) (end 137.59588 105.41) (width 0.3) (layer B.Cu) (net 12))
 (segment (start 128.223 98.23) (end 131.631 98.23) (width 0.3) (layer B.Cu) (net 12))
 (segment (start 131.631 98.23) (end 135.70749 102.30649) (width 0.3) (layer B.Cu) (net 12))
 (segment (start 139.065 106.68) (end 140.335 105.41) (width 0.3) (layer B.Cu) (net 11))
 (segment (start 131.35176 98.73) (end 135.20748 102.58572) (width 0.3) (layer B.Cu) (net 11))
 (segment (start 135.20748 104.72748) (end 137.16 106.68) (width 0.3) (layer B.Cu) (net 11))
 (segment (start 135.20748 102.58572) (end 135.20748 104.72748) (width 0.3) (layer B.Cu) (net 11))
 (segment (start 128.223 98.73) (end 131.35176 98.73) (width 0.3) (layer B.Cu) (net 11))
 (segment (start 137.16 106.68) (end 139.065 106.68) (width 0.3) (layer B.Cu) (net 11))
 (segment (start 137.6045 107.95) (end 137.795 107.95) (width 0.3) (layer B.Cu) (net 10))
 (segment (start 134.70747 105.05297) (end 137.6045 107.95) (width 0.3) (layer B.Cu) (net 10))
 (segment (start 134.70747 102.79283) (end 134.70747 105.05297) (width 0.3) (layer B.Cu) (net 10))
 (segment (start 128.223 99.23) (end 131.14464 99.23) (width 0.3) (layer B.Cu) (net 10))
 (segment (start 131.14464 99.23) (end 134.70747 102.79283) (width 0.3) (layer B.Cu) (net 10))
 (segment (start 139.065 109.22) (end 140.335 107.95) (width 0.3) (layer B.Cu) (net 9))
 (segment (start 130.93752 99.73) (end 134.20746 102.99994) (width 0.3) (layer B.Cu) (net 9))
 (segment (start 134.20746 106.33096) (end 137.0965 109.22) (width 0.3) (layer B.Cu) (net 9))
 (segment (start 128.223 99.73) (end 130.93752 99.73) (width 0.3) (layer B.Cu) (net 9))
 (segment (start 134.20746 102.99994) (end 134.20746 106.33096) (width 0.3) (layer B.Cu) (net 9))
 (segment (start 137.0965 109.22) (end 139.065 109.22) (width 0.3) (layer B.Cu) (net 9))
 (segment (start 128.223 100.23) (end 130.7304 100.23) (width 0.3) (layer B.Cu) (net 8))
 (segment (start 133.70745 106.60157) (end 137.59588 110.49) (width 0.3) (layer B.Cu) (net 8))
 (segment (start 130.7304 100.23) (end 133.70745 103.20705) (width 0.3) (layer B.Cu) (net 8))
 (segment (start 137.59588 110.49) (end 137.795 110.49) (width 0.3) (layer B.Cu) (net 8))
 (segment (start 133.70745 103.20705) (end 133.70745 106.60157) (width 0.3) (layer B.Cu) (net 8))
 (segment (start 128.223 100.73) (end 130.52328 100.73) (width 0.3) (layer B.Cu) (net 7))
 (segment (start 130.52328 100.73) (end 133.20744 103.41416) (width 0.3) (layer B.Cu) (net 7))
 (segment (start 133.20744 107.678442) (end 137.288998 111.76) (width 0.3) (layer B.Cu) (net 7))
 (segment (start 133.20744 103.41416) (end 133.20744 107.678442) (width 0.3) (layer B.Cu) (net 7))
 (segment (start 139.065 111.76) (end 140.335 110.49) (width 0.3) (layer B.Cu) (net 7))
 (segment (start 137.288998 111.76) (end 139.065 111.76) (width 0.3) (layer B.Cu) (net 7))
 (segment (start 128.223 101.23) (end 130.31616 101.23) (width 0.3) (layer B.Cu) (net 6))
 (segment (start 130.31616 101.23) (end 132.70743 103.62127) (width 0.3) (layer B.Cu) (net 6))
 (segment (start 132.70743 107.94243) (end 137.795 113.03) (width 0.3) (layer B.Cu) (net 6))
 (segment (start 132.70743 103.62127) (end 132.70743 107.94243) (width 0.3) (layer B.Cu) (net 6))
 (segment (start 128.223 101.73) (end 130.10904 101.73) (width 0.3) (layer B.Cu) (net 5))
 (segment (start 130.10904 101.73) (end 132.20742 103.82838) (width 0.3) (layer B.Cu) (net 5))
 (segment (start 132.20742 109.218422) (end 137.288998 114.3) (width 0.3) (layer B.Cu) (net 5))
 (segment (start 132.20742 103.82838) (end 132.20742 109.218422) (width 0.3) (layer B.Cu) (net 5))
 (segment (start 139.065 114.3) (end 140.335 113.03) (width 0.3) (layer B.Cu) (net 5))
 (segment (start 137.288998 114.3) (end 139.065 114.3) (width 0.3) (layer B.Cu) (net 5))
 (segment (start 128.223 102.23) (end 129.90192 102.23) (width 0.3) (layer B.Cu) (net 4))
 (segment (start 131.70741 109.48241) (end 137.795 115.57) (width 0.3) (layer B.Cu) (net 4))
 (segment (start 129.90192 102.23) (end 131.70741 104.03549) (width 0.3) (layer B.Cu) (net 4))
 (segment (start 131.70741 104.03549) (end 131.70741 109.48241) (width 0.3) (layer B.Cu) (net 4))
 (segment (start 129.6948 102.73) (end 128.223 102.73) (width 0.3) (layer B.Cu) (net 3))
 (segment (start 139.065 116.84) (end 137.288998 116.84) (width 0.3) (layer B.Cu) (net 3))
 (segment (start 131.191 110.742002) (end 131.191 104.2262) (width 0.3) (layer B.Cu) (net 3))
 (segment (start 140.335 115.57) (end 139.065 116.84) (width 0.3) (layer B.Cu) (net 3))
 (segment (start 137.288998 116.84) (end 131.191 110.742002) (width 0.3) (layer B.Cu) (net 3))
 (segment (start 131.191 104.2262) (end 129.6948 102.73) (width 0.3) (layer B.Cu) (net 3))
 (segment (start 129.48768 103.23) (end 128.223 103.23) (width 0.3) (layer B.Cu) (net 2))
 (segment (start 130.683 104.42532) (end 129.48768 103.23) (width 0.3) (layer B.Cu) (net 2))
 (segment (start 137.795 118.11) (end 130.683 110.998) (width 0.3) (layer B.Cu) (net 2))
 (segment (start 130.683 110.998) (end 130.683 104.42532) (width 0.3) (layer B.Cu) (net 2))
 (segment (start 129.1935 103.73) (end 128.223 103.73) (width 0.3) (layer B.Cu) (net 1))
 (segment (start 130.1115 104.648) (end 129.1935 103.73) (width 0.3) (layer B.Cu) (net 1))
 (segment (start 139.0015 119.4435) (end 137.2235 119.4435) (width 0.3) (layer B.Cu) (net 1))
 (segment (start 130.1115 111.1885) (end 130.1115 104.648) (width 0.3) (layer B.Cu) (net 1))
 (segment (start 140.335 118.11) (end 139.0015 119.4435) (width 0.3) (layer B.Cu) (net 1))
 (segment (start 136.2075 117.2845) (end 130.1115 111.1885) (width 0.3) (layer B.Cu) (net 1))
 (segment (start 137.2235 119.4435) (end 136.2075 118.4275) (width 0.3) (layer B.Cu) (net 1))
 (segment (start 136.2075 118.4275) (end 136.2075 117.2845) (width 0.3) (layer B.Cu) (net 1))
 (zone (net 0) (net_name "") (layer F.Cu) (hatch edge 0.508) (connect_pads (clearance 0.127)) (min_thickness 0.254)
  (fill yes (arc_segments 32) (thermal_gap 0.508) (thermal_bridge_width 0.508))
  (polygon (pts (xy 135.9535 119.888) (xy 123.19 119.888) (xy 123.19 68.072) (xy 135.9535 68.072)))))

